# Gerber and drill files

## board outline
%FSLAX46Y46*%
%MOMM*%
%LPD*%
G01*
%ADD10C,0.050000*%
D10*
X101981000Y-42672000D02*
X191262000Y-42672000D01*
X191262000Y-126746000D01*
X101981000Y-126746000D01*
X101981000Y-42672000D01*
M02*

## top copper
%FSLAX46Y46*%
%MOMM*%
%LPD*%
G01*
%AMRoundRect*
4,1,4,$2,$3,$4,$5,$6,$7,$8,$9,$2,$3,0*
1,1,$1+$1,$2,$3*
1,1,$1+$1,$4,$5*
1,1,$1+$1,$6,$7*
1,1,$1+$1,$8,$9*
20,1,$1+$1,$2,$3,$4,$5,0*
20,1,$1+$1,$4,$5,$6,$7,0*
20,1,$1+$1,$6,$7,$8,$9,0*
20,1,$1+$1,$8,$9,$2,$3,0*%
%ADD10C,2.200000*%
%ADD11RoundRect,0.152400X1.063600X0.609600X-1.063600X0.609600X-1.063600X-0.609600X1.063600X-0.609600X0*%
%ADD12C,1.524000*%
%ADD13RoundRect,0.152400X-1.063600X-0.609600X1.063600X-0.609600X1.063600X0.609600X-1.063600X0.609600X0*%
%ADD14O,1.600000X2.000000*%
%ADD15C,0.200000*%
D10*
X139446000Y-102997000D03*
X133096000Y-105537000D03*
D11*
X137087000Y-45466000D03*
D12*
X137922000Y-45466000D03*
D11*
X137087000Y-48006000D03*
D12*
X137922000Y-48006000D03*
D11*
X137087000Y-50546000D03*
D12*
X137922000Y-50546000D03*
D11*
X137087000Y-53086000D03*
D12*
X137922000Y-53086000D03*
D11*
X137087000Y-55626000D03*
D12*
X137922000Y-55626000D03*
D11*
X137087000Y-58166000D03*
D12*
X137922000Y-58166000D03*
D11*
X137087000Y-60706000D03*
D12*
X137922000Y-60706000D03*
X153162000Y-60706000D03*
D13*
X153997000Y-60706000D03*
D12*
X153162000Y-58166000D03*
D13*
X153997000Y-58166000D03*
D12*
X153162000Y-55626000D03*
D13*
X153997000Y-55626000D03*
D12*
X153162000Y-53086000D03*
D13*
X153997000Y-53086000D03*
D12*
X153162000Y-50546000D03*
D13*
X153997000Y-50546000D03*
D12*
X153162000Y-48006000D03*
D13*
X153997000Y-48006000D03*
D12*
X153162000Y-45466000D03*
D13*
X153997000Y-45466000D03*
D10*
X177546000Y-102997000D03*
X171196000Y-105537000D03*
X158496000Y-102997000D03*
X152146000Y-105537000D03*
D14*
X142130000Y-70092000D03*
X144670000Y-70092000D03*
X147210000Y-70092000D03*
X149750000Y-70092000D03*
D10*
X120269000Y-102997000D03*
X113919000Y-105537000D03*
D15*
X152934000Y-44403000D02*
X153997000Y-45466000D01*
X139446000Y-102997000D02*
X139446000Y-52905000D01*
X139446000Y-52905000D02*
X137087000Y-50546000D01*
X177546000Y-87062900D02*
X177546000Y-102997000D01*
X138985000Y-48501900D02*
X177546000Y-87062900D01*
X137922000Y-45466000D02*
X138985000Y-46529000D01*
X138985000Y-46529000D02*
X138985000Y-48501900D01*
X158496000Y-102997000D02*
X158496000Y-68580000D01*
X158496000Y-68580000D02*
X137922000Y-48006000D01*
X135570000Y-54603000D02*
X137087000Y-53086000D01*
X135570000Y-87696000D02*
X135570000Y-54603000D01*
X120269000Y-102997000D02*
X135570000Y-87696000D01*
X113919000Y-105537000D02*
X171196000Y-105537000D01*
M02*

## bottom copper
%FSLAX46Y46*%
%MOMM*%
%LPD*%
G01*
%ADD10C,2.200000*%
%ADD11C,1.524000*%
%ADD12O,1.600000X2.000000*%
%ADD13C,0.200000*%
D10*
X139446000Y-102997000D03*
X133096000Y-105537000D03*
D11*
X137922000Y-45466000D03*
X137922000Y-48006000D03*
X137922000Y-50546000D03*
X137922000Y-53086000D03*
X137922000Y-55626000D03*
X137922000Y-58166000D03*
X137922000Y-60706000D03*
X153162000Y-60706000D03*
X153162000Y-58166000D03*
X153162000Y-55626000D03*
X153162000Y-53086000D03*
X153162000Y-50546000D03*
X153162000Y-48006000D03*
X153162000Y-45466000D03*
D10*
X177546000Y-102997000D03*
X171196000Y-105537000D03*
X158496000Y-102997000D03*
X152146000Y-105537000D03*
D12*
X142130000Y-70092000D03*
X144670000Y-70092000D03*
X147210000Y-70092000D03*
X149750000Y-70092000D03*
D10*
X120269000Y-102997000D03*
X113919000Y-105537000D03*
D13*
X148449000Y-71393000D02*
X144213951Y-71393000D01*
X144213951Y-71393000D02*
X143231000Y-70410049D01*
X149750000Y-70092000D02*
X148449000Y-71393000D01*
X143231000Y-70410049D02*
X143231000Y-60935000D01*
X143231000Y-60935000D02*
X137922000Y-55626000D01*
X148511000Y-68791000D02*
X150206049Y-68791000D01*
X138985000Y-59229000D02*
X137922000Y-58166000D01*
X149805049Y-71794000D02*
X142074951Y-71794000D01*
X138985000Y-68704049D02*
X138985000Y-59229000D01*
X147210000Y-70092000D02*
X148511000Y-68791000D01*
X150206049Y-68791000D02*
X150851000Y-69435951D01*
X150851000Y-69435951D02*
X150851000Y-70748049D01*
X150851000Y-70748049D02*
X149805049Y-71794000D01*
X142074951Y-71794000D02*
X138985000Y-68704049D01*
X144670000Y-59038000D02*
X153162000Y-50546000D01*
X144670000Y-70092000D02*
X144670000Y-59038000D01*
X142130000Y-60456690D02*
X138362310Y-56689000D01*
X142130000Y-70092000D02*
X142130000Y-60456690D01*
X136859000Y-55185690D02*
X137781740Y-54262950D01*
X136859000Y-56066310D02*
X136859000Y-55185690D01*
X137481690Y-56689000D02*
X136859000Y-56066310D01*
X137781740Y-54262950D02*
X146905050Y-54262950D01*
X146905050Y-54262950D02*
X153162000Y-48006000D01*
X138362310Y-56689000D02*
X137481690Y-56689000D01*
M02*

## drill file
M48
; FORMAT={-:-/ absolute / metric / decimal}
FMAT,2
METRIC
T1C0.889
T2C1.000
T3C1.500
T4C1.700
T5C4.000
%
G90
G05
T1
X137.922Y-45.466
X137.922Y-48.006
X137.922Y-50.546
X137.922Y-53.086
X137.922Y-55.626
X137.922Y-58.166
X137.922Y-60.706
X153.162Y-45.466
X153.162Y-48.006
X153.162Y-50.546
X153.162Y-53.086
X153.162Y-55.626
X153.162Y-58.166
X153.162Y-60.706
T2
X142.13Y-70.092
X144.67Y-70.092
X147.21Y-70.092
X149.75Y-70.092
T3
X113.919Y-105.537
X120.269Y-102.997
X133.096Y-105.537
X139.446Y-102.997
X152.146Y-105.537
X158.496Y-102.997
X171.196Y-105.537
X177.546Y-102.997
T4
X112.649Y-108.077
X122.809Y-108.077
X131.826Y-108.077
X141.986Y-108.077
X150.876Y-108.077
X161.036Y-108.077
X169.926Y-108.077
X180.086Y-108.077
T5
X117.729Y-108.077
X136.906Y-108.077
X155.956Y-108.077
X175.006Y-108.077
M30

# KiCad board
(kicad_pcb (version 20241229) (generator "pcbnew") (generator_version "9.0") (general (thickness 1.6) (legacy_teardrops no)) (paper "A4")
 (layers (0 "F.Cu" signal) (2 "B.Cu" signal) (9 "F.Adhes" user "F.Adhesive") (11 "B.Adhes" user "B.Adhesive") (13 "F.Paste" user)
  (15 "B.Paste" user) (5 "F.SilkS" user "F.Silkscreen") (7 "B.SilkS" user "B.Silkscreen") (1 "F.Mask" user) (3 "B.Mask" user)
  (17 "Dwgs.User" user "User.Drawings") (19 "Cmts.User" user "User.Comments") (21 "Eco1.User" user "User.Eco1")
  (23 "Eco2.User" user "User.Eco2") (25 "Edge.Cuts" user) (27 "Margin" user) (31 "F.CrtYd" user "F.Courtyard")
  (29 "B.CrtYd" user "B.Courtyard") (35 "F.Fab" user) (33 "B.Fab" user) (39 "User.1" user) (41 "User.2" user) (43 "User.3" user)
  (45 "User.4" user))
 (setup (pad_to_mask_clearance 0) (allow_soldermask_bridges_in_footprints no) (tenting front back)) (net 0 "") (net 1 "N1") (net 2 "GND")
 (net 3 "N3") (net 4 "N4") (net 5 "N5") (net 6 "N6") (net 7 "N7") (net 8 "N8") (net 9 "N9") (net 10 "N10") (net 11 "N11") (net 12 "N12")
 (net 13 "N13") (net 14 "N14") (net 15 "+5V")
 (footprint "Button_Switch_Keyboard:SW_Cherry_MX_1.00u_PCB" (layer "F.Cu") (at 139.446 102.997)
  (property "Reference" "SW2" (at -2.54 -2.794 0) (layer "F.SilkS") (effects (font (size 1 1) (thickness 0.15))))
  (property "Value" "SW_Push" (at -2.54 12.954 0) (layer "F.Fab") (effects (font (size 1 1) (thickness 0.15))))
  (pad "" np_thru_hole circle (at -7.62 5.08) (size 1.7 1.7) (drill 1.7) (layers "*.Cu" "*.Mask"))
  (pad "" np_thru_hole circle (at -2.54 5.08) (size 4 4) (drill 4) (layers "*.Cu" "*.Mask"))
  (pad "" np_thru_hole circle (at 2.54 5.08) (size 1.7 1.7) (drill 1.7) (layers "*.Cu" "*.Mask"))
  (pad "1" thru_hole circle (at 0 0) (size 2.2 2.2) (drill 1.5) (layers "*.Cu" "*.Mask") (remove_unused_layers no) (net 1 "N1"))
  (pad "2" thru_hole circle (at -6.35 2.54) (size 2.2 2.2) (drill 1.5) (layers "*.Cu" "*.Mask") (remove_unused_layers no) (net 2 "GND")))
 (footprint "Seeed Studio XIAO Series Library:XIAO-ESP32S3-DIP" (layer "F.Cu") (at 145.542 53.086)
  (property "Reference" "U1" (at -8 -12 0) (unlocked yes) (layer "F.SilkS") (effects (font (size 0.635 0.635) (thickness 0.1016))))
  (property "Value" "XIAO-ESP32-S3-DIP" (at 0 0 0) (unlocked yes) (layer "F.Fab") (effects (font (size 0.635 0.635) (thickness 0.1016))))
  (pad "1" smd roundrect (at -8.455 -7.62 180) (size 2.432 1.524) (layers "F.Cu" "F.Mask") (roundrect_rratio 0.1) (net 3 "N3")
   (thermal_bridge_angle 45))
  (pad "1" thru_hole circle (at -7.62 -7.62 180) (size 1.524 1.524) (drill 0.889) (layers "*.Cu" "*.Mask") (remove_unused_layers no)
   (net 3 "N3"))
  (pad "2" smd roundrect (at -8.455 -5.08 180) (size 2.432 1.524) (layers "F.Cu" "F.Mask") (roundrect_rratio 0.1) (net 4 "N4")
   (thermal_bridge_angle 45))
  (pad "2" thru_hole circle (at -7.62 -5.08 180) (size 1.524 1.524) (drill 0.889) (layers "*.Cu" "*.Mask") (remove_unused_layers no)
   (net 4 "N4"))
  (pad "3" smd roundrect (at -8.455 -2.54 180) (size 2.432 1.524) (layers "F.Cu" "F.Mask") (roundrect_rratio 0.1) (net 1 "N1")
   (thermal_bridge_angle 45))
  (pad "3" thru_hole circle (at -7.62 -2.54 180) (size 1.524 1.524) (drill 0.889) (layers "*.Cu" "*.Mask") (remove_unused_layers no)
   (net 1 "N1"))
  (pad "4" smd roundrect (at -8.455 0 180) (size 2.432 1.524) (layers "F.Cu" "F.Mask") (roundrect_rratio 0.1) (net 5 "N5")
   (thermal_bridge_angle 45))
  (pad "4" thru_hole circle (at -7.62 0 180) (size 1.524 1.524) (drill 0.889) (layers "*.Cu" "*.Mask") (remove_unused_layers no)
   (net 5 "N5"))
  (pad "5" smd roundrect (at -8.455 2.54 180) (size 2.432 1.524) (layers "F.Cu" "F.Mask") (roundrect_rratio 0.1) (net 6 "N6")
   (thermal_bridge_angle 45))
  (pad "5" thru_hole circle (at -7.62 2.54 180) (size 1.524 1.524) (drill 0.889) (layers "*.Cu" "*.Mask") (remove_unused_layers no)
   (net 6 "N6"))
  (pad "6" smd roundrect (at -8.455 5.08 180) (size 2.432 1.524) (layers "F.Cu" "F.Mask") (roundrect_rratio 0.1) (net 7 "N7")
   (thermal_bridge_angle 45))
  (pad "6" thru_hole circle (at -7.62 5.08 180) (size 1.524 1.524) (drill 0.889) (layers "*.Cu" "*.Mask") (remove_unused_layers no)
   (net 7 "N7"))
  (pad "7" smd roundrect (at -8.455 7.62 180) (size 2.432 1.524) (layers "F.Cu" "F.Mask") (roundrect_rratio 0.1) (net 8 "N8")
   (thermal_bridge_angle 45))
  (pad "7" thru_hole circle (at -7.62 7.62 180) (size 1.524 1.524) (drill 0.889) (layers "*.Cu" "*.Mask") (remove_unused_layers no)
   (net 8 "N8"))
  (pad "8" thru_hole circle (at 7.62 7.62) (size 1.524 1.524) (drill 0.889) (layers "*.Cu" "*.Mask") (remove_unused_layers no) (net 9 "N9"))
  (pad "8" smd roundrect (at 8.455 7.62) (size 2.432 1.524) (layers "F.Cu" "F.Mask") (roundrect_rratio 0.1) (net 9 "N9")
   (thermal_bridge_angle 45))
  (pad "9" thru_hole circle (at 7.62 5.08) (size 1.524 1.524) (drill 0.889) (layers "*.Cu" "*.Mask") (remove_unused_layers no)
   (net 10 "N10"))
  (pad "9" smd roundrect (at 8.455 5.08) (size 2.432 1.524) (layers "F.Cu" "F.Mask") (roundrect_rratio 0.1) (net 10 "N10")
   (thermal_bridge_angle 45))
  (pad "10" thru_hole circle (at 7.62 2.54) (size 1.524 1.524) (drill 0.889) (layers "*.Cu" "*.Mask") (remove_unused_layers no)
   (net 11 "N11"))
  (pad "10" smd roundrect (at 8.455 2.54) (size 2.432 1.524) (layers "F.Cu" "F.Mask") (roundrect_rratio 0.1) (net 11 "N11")
   (thermal_bridge_angle 45))
  (pad "11" thru_hole circle (at 7.62 0) (size 1.524 1.524) (drill 0.889) (layers "*.Cu" "*.Mask") (remove_unused_layers no) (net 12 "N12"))
  (pad "11" smd roundrect (at 8.455 0) (size 2.432 1.524) (layers "F.Cu" "F.Mask") (roundrect_rratio 0.1) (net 12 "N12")
   (thermal_bridge_angle 45))
  (pad "12" thru_hole circle (at 7.62 -2.54) (size 1.524 1.524) (drill 0.889) (layers "*.Cu" "*.Mask") (remove_unused_layers no)
   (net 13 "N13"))
  (pad "12" smd roundrect (at 8.455 -2.54) (size 2.432 1.524) (layers "F.Cu" "F.Mask") (roundrect_rratio 0.1) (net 13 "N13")
   (thermal_bridge_angle 45))
  (pad "13" thru_hole circle (at 7.62 -5.08) (size 1.524 1.524) (drill 0.889) (layers "*.Cu" "*.Mask") (remove_unused_layers no)
   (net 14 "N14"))
  (pad "13" smd roundrect (at 8.455 -5.08) (size 2.432 1.524) (layers "F.Cu" "F.Mask") (roundrect_rratio 0.1) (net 14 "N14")
   (thermal_bridge_angle 45))
  (pad "14" thru_hole circle (at 7.62 -7.62) (size 1.524 1.524) (drill 0.889) (layers "*.Cu" "*.Mask") (remove_unused_layers no)
   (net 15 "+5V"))
  (pad "14" smd roundrect (at 8.455 -7.62) (size 2.432 1.524) (layers "F.Cu" "F.Mask") (roundrect_rratio 0.1) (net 15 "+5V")
   (thermal_bridge_angle 45)))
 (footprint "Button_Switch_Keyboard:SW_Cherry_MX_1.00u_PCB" (layer "F.Cu") (at 177.546 102.997)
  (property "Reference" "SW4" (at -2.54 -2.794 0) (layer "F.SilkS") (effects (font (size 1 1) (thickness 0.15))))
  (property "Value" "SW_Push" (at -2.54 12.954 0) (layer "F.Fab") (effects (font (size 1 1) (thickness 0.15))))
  (pad "" np_thru_hole circle (at -7.62 5.08) (size 1.7 1.7) (drill 1.7) (layers "*.Cu" "*.Mask"))
  (pad "" np_thru_hole circle (at -2.54 5.08) (size 4 4) (drill 4) (layers "*.Cu" "*.Mask"))
  (pad "" np_thru_hole circle (at 2.54 5.08) (size 1.7 1.7) (drill 1.7) (layers "*.Cu" "*.Mask"))
  (pad "1" thru_hole circle (at 0 0) (size 2.2 2.2) (drill 1.5) (layers "*.Cu" "*.Mask") (remove_unused_layers no) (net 3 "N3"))
  (pad "2" thru_hole circle (at -6.35 2.54) (size 2.2 2.2) (drill 1.5) (layers "*.Cu" "*.Mask") (remove_unused_layers no) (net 2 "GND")))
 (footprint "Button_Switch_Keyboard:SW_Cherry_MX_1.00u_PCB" (layer "F.Cu") (at 158.496 102.997)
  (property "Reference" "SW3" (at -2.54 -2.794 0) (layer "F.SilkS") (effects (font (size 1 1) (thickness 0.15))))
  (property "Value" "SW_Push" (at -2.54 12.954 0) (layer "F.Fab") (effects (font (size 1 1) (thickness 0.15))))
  (pad "" np_thru_hole circle (at -7.62 5.08) (size 1.7 1.7) (drill 1.7) (layers "*.Cu" "*.Mask"))
  (pad "" np_thru_hole circle (at -2.54 5.08) (size 4 4) (drill 4) (layers "*.Cu" "*.Mask"))
  (pad "" np_thru_hole circle (at 2.54 5.08) (size 1.7 1.7) (drill 1.7) (layers "*.Cu" "*.Mask"))
  (pad "1" thru_hole circle (at 0 0) (size 2.2 2.2) (drill 1.5) (layers "*.Cu" "*.Mask") (remove_unused_layers no) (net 4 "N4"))
  (pad "2" thru_hole circle (at -6.35 2.54) (size 2.2 2.2) (drill 1.5) (layers "*.Cu" "*.Mask") (remove_unused_layers no) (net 2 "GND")))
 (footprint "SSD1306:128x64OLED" (layer "F.Cu") (at 145.75 80.692)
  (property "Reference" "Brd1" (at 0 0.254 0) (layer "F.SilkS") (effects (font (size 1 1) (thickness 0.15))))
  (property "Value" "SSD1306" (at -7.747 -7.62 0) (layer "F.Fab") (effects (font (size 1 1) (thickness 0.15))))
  (pad "1" thru_hole oval (at -3.62 -10.6 90) (size 2 1.6) (drill 1) (layers "*.Cu" "*.Mask") (remove_unused_layers no) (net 14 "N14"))
  (pad "2" thru_hole oval (at -1.08 -10.6 90) (size 2 1.6) (drill 1) (layers "*.Cu" "*.Mask") (remove_unused_layers no) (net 13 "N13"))
  (pad "3" thru_hole oval (at 1.46 -10.6 90) (size 2 1.6) (drill 1) (layers "*.Cu" "*.Mask") (remove_unused_layers no) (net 7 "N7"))
  (pad "4" thru_hole oval (at 4 -10.6 90) (size 2 1.6) (drill 1) (layers "*.Cu" "*.Mask") (remove_unused_layers no) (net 6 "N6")))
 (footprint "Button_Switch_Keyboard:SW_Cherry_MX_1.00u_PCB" (layer "F.Cu") (at 120.269 102.997)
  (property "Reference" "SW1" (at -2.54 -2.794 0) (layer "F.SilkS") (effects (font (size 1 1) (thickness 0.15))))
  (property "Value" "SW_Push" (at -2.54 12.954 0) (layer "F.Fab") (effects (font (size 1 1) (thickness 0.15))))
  (pad "" np_thru_hole circle (at -7.62 5.08) (size 1.7 1.7) (drill 1.7) (layers "*.Cu" "*.Mask"))
  (pad "" np_thru_hole circle (at -2.54 5.08) (size 4 4) (drill 4) (layers "*.Cu" "*.Mask"))
  (pad "" np_thru_hole circle (at 2.54 5.08) (size 1.7 1.7) (drill 1.7) (layers "*.Cu" "*.Mask"))
  (pad "1" thru_hole circle (at 0 0) (size 2.2 2.2) (drill 1.5) (layers "*.Cu" "*.Mask") (remove_unused_layers no) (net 5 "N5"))
  (pad "2" thru_hole circle (at -6.35 2.54) (size 2.2 2.2) (drill 1.5) (layers "*.Cu" "*.Mask") (remove_unused_layers no) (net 2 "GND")))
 (gr_rect (start 101.981 42.672) (end 191.262 126.746) (stroke (width 0.05) (type default)) (fill no) (layer "Edge.Cuts"))
 (segment (start 148.449 71.393) (end 144.213951 71.393) (width 0.2) (layer "B.Cu") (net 6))
 (segment (start 144.213951 71.393) (end 143.231 70.410049) (width 0.2) (layer "B.Cu") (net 6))
 (segment (start 149.75 70.092) (end 148.449 71.393) (width 0.2) (layer "B.Cu") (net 6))
 (segment (start 143.231 70.410049) (end 143.231 60.935) (width 0.2) (layer "B.Cu") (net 6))
 (segment (start 143.231 60.935) (end 137.922 55.626) (width 0.2) (layer "B.Cu") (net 6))
 (segment (start 148.511 68.791) (end 150.206049 68.791) (width 0.2) (layer "B.Cu") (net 7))
 (segment (start 138.985 59.229) (end 137.922 58.166) (width 0.2) (layer "B.Cu") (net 7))
 (segment (start 149.805049 71.794) (end 142.074951 71.794) (width 0.2) (layer "B.Cu") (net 7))
 (segment (start 138.985 68.704049) (end 138.985 59.229) (width 0.2) (layer "B.Cu") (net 7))
 (segment (start 147.21 70.092) (end 148.511 68.791) (width 0.2) (layer "B.Cu") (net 7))
 (segment (start 150.206049 68.791) (end 150.851 69.435951) (width 0.2) (layer "B.Cu") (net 7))
 (segment (start 150.851 69.435951) (end 150.851 70.748049) (width 0.2) (layer "B.Cu") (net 7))
 (segment (start 150.851 70.748049) (end 149.805049 71.794) (width 0.2) (layer "B.Cu") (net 7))
 (segment (start 142.074951 71.794) (end 138.985 68.704049) (width 0.2) (layer "B.Cu") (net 7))
 (segment (start 144.67 59.038) (end 153.162 50.546) (width 0.2) (layer "B.Cu") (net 13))
 (segment (start 144.67 70.092) (end 144.67 59.038) (width 0.2) (layer "B.Cu") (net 13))
 (segment (start 142.13 60.45669) (end 138.36231 56.689) (width 0.2) (layer "B.Cu") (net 14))
 (segment (start 142.13 70.092) (end 142.13 60.45669) (width 0.2) (layer "B.Cu") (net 14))
 (segment (start 136.859 55.18569) (end 137.78174 54.26295) (width 0.2) (layer "B.Cu") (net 14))
 (segment (start 136.859 56.06631) (end 136.859 55.18569) (width 0.2) (layer "B.Cu") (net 14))
 (segment (start 137.48169 56.689) (end 136.859 56.06631) (width 0.2) (layer "B.Cu") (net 14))
 (segment (start 137.78174 54.26295) (end 146.90505 54.26295) (width 0.2) (layer "B.Cu") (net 14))
 (segment (start 146.90505 54.26295) (end 153.162 48.006) (width 0.2) (layer "B.Cu") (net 14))
 (segment (start 138.36231 56.689) (end 137.48169 56.689) (width 0.2) (layer "B.Cu") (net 14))
 (segment (start 152.934 44.403) (end 153.997 45.466) (width 0.2) (layer "F.Cu") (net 15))
 (segment (start 139.446 102.997) (end 139.446 52.905) (width 0.2) (layer "F.Cu") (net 1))
 (segment (start 139.446 52.905) (end 137.087 50.546) (width 0.2) (layer "F.Cu") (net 1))
 (segment (start 177.546 87.0629) (end 177.546 102.997) (width 0.2) (layer "F.Cu") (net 3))
 (segment (start 138.985 48.5019) (end 177.546 87.0629) (width 0.2) (layer "F.Cu") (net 3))
 (segment (start 137.922 45.466) (end 138.985 46.529) (width 0.2) (layer "F.Cu") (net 3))
 (segment (start 138.985 46.529) (end 138.985 48.5019) (width 0.2) (layer "F.Cu") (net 3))
 (segment (start 158.496 102.997) (end 158.496 68.58) (width 0.2) (layer "F.Cu") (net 4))
 (segment (start 158.496 68.58) (end 137.922 48.006) (width 0.2) (layer "F.Cu") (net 4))
 (segment (start 135.57 54.603) (end 137.087 53.086) (width 0.2) (layer "F.Cu") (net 5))
 (segment (start 135.57 87.696) (end 135.57 54.603) (width 0.2) (layer "F.Cu") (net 5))
 (segment (start 120.269 102.997) (end 135.57 87.696) (width 0.2) (layer "F.Cu") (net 5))
 (segment (start 113.919 105.537) (end 171.196 105.537) (width 0.2) (layer "F.Cu") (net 2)))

